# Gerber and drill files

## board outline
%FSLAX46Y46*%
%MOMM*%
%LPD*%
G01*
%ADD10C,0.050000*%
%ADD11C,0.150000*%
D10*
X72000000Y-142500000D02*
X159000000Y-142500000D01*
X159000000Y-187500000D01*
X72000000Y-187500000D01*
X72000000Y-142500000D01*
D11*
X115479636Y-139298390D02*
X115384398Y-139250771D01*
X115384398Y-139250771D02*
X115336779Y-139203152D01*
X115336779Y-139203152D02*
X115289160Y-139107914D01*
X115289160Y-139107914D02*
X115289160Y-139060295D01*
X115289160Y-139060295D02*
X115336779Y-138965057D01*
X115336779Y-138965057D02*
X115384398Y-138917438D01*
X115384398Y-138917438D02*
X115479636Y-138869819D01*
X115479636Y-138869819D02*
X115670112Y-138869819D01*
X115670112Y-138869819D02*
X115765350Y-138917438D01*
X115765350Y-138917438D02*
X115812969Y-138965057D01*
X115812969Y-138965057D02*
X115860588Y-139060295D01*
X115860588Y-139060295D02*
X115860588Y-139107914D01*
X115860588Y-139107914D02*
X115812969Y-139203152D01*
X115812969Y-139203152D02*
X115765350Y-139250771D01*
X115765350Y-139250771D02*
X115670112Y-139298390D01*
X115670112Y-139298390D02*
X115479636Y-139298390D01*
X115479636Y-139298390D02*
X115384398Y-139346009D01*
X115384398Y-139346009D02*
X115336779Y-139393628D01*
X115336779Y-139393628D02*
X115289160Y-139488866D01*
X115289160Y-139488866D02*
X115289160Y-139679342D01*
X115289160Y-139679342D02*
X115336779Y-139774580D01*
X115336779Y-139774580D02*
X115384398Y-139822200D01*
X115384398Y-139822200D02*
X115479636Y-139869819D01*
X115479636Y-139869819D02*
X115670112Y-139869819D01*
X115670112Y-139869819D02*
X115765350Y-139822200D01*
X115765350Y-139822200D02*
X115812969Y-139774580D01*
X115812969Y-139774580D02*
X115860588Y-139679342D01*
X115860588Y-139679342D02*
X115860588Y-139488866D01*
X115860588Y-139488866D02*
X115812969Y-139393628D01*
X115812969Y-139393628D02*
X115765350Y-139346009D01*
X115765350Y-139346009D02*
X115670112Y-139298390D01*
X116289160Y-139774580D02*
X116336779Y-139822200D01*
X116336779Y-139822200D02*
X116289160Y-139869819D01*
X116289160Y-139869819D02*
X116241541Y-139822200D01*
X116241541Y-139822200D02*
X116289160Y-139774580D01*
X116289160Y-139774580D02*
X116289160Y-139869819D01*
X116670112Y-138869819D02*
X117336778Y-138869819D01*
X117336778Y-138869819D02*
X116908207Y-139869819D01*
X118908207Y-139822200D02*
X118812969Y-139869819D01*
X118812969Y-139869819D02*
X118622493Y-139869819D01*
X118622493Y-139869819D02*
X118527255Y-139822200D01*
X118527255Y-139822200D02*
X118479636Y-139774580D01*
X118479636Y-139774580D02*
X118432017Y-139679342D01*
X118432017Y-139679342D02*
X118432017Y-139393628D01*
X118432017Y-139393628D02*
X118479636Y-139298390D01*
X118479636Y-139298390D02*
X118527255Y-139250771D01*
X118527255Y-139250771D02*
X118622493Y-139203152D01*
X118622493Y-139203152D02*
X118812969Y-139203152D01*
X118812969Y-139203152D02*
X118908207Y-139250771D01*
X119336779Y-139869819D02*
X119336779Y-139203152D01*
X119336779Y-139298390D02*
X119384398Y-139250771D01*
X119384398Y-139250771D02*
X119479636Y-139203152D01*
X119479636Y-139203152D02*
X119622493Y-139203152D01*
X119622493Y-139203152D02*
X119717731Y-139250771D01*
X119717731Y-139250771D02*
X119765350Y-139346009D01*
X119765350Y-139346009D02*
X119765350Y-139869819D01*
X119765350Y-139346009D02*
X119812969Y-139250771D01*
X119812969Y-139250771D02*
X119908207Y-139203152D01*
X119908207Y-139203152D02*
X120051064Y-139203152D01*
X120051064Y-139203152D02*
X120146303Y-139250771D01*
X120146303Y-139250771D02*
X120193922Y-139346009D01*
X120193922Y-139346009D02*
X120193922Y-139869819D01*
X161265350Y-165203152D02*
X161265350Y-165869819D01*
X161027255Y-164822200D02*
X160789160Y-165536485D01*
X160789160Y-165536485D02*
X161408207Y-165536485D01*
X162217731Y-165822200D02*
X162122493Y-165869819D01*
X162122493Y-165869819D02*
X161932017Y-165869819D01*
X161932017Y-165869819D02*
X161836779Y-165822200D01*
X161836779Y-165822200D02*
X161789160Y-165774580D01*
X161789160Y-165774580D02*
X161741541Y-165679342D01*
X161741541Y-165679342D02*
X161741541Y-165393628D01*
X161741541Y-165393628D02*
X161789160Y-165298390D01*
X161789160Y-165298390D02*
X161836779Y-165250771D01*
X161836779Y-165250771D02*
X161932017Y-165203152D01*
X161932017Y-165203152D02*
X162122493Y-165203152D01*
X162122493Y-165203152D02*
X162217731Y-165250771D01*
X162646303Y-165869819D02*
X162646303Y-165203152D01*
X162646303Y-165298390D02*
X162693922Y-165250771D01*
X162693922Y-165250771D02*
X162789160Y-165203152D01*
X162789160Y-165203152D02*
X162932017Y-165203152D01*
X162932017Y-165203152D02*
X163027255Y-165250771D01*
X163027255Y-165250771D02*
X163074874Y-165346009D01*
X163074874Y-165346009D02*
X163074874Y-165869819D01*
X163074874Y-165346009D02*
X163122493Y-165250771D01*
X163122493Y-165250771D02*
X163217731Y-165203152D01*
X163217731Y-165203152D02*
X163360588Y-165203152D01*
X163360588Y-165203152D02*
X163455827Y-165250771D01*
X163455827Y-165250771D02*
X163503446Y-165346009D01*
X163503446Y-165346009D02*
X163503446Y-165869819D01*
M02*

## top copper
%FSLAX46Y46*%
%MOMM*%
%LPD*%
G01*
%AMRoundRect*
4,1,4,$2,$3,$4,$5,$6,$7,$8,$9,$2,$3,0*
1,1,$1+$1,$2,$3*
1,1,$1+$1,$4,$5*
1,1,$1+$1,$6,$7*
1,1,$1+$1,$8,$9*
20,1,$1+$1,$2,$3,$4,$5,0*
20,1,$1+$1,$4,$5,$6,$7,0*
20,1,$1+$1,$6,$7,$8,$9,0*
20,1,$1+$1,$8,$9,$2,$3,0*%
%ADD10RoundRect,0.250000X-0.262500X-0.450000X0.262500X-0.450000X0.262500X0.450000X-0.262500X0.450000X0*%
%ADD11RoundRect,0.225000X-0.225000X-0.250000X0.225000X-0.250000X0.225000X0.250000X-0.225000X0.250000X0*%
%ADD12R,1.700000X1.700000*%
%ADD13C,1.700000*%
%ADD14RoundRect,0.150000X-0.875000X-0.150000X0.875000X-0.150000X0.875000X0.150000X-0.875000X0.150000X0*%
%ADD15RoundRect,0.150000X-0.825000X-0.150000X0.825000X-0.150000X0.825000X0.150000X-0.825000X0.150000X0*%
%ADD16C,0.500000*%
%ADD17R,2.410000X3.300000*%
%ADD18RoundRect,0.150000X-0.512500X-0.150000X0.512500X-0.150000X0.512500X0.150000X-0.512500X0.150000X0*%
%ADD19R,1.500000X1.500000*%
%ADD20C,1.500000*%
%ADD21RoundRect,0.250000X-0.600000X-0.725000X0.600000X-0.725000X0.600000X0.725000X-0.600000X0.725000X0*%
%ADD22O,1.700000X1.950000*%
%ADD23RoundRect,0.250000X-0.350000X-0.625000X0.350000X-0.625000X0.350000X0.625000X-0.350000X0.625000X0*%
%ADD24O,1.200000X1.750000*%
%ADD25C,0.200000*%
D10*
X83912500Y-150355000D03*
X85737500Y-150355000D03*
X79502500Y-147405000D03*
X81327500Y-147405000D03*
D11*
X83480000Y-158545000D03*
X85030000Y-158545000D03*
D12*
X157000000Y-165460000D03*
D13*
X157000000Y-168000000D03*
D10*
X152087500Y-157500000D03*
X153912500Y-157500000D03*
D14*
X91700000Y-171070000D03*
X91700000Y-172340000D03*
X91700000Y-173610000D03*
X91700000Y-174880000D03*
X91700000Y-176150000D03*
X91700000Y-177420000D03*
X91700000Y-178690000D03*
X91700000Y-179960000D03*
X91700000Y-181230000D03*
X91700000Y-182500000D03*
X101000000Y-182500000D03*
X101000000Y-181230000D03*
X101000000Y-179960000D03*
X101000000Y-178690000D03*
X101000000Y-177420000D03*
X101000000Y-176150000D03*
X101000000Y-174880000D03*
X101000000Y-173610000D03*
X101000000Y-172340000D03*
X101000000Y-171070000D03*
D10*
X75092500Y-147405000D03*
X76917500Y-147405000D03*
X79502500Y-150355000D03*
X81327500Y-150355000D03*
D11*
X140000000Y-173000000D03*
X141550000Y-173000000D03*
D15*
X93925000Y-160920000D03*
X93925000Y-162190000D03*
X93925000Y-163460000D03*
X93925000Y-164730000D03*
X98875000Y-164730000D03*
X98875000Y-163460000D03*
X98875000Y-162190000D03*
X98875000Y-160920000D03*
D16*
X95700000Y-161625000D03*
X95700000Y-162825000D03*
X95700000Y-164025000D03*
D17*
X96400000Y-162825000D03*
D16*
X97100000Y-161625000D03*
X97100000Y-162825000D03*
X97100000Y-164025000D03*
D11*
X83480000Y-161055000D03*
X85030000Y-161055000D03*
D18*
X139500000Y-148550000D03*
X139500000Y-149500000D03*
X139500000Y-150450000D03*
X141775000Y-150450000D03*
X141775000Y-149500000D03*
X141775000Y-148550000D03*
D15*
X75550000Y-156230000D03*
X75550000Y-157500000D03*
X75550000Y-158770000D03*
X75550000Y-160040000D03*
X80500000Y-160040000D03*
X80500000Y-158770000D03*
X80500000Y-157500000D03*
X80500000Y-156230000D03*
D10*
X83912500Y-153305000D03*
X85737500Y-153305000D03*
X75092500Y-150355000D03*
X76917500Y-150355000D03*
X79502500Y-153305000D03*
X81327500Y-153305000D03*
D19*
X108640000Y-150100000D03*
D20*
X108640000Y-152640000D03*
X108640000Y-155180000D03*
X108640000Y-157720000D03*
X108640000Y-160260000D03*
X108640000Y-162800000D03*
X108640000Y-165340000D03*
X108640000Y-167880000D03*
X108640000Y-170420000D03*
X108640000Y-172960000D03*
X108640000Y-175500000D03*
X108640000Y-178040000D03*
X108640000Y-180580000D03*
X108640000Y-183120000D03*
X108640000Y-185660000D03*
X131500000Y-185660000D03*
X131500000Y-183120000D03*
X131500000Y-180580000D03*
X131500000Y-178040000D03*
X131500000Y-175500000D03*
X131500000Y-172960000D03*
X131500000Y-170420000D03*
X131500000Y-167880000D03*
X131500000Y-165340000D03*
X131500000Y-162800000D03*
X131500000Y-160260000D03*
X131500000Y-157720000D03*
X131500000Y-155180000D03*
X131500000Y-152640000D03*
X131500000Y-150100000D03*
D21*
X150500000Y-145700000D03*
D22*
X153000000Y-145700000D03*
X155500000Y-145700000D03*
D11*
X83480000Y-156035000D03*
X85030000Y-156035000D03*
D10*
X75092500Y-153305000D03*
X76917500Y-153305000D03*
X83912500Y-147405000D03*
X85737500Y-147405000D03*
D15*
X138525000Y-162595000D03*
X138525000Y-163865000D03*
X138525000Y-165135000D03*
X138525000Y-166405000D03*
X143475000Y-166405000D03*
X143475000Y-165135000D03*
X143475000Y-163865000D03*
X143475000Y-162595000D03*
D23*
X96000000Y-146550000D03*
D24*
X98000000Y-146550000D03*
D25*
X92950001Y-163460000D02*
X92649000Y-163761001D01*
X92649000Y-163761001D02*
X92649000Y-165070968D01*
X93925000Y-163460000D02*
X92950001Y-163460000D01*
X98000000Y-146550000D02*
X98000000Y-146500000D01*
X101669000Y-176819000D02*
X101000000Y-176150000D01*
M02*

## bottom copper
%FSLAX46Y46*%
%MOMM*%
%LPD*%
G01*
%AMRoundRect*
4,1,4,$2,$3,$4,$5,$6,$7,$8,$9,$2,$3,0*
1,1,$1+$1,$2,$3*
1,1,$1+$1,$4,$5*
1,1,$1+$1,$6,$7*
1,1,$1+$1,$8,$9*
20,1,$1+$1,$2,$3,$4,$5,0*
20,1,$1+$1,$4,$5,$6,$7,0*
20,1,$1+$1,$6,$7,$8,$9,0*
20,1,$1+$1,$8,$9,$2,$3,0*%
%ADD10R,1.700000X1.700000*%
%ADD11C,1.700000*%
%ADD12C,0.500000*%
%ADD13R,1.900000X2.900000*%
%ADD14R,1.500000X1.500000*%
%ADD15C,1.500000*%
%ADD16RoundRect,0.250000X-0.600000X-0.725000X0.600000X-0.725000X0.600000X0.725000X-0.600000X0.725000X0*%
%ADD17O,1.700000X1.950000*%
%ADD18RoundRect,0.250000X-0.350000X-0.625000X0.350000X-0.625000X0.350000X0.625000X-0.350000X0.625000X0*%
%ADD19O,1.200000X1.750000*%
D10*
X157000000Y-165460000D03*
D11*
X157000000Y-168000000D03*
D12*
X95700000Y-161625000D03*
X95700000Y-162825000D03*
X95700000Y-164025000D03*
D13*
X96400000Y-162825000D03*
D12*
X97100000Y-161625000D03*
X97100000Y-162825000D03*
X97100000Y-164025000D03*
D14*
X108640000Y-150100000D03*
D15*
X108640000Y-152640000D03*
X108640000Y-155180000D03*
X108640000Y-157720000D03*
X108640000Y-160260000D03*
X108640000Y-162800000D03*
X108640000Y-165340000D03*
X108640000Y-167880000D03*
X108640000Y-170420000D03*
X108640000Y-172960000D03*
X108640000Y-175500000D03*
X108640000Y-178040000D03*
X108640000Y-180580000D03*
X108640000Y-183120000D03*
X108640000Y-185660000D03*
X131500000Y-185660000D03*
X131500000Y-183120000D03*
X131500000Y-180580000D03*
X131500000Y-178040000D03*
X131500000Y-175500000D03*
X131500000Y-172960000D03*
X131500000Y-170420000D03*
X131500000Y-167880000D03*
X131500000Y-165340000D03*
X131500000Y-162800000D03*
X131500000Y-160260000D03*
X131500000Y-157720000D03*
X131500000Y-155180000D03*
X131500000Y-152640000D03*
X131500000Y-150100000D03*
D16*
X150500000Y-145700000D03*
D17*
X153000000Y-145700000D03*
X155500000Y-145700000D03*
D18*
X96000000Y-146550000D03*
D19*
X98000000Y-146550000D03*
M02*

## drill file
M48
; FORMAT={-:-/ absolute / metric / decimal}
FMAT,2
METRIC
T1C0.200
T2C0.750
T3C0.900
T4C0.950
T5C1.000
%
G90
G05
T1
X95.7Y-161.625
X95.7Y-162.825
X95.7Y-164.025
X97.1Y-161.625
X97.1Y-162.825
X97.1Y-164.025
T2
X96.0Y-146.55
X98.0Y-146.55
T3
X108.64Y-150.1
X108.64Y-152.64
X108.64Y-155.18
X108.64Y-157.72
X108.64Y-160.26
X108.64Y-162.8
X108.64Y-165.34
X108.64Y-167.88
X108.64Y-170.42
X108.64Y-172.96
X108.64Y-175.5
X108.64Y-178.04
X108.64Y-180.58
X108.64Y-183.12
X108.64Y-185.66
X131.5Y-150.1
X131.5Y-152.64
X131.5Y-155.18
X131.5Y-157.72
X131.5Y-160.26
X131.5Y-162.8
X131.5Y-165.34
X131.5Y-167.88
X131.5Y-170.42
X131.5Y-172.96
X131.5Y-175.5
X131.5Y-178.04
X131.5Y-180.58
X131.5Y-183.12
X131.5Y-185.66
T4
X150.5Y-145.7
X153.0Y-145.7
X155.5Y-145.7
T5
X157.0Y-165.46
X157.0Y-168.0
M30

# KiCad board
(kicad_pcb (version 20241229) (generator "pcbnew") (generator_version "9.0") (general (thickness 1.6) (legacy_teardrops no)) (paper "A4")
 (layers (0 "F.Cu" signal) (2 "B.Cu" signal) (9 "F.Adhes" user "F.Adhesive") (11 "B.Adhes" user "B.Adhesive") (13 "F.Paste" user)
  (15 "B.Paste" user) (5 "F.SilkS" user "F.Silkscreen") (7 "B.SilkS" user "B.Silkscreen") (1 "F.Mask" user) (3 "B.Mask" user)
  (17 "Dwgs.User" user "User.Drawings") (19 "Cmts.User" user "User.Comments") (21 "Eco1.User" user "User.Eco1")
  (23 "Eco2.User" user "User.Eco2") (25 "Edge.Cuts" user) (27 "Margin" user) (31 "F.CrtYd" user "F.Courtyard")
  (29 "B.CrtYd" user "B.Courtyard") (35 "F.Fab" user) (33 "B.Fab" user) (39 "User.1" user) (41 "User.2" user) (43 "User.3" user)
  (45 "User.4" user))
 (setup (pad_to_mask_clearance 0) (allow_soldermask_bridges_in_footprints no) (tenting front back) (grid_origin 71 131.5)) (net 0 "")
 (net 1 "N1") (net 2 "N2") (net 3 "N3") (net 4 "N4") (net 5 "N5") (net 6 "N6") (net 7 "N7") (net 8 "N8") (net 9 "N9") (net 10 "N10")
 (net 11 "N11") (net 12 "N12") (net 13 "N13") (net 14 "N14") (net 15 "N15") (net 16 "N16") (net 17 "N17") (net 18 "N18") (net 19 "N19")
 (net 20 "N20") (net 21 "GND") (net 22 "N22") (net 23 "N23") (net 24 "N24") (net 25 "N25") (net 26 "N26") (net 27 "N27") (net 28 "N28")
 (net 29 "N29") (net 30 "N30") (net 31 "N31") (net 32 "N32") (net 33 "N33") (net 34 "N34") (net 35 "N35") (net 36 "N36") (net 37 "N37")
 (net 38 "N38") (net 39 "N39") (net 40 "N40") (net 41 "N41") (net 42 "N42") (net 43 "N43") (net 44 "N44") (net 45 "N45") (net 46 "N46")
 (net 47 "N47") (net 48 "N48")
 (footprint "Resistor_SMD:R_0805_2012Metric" (layer "F.Cu") (at 84.825 150.355)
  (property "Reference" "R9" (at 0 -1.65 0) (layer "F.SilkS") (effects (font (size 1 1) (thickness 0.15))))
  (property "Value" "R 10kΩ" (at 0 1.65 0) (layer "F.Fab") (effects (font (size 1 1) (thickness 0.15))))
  (pad "1" smd roundrect (at -0.9125 0) (size 1.025 1.4) (layers "F.Cu" "F.Mask" "F.Paste") (roundrect_rratio 0.243902) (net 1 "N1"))
  (pad "2" smd roundrect (at 0.9125 0) (size 1.025 1.4) (layers "F.Cu" "F.Mask" "F.Paste") (roundrect_rratio 0.243902) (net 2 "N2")))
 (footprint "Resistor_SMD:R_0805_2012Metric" (layer "F.Cu") (at 80.415 147.405)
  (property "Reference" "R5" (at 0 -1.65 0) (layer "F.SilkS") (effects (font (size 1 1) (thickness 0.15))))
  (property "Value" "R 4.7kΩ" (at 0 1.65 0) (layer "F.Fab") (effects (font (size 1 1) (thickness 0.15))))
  (pad "1" smd roundrect (at -0.9125 0) (size 1.025 1.4) (layers "F.Cu" "F.Mask" "F.Paste") (roundrect_rratio 0.243902) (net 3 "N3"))
  (pad "2" smd roundrect (at 0.9125 0) (size 1.025 1.4) (layers "F.Cu" "F.Mask" "F.Paste") (roundrect_rratio 0.243902) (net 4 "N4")))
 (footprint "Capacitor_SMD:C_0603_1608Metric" (layer "F.Cu") (at 84.255 158.545)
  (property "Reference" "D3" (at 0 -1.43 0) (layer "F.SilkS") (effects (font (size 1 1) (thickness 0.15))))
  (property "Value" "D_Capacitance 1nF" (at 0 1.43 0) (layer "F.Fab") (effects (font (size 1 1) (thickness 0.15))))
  (pad "1" smd roundrect (at -0.775 0) (size 0.9 0.95) (layers "F.Cu" "F.Mask" "F.Paste") (roundrect_rratio 0.25) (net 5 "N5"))
  (pad "2" smd roundrect (at 0.775 0) (size 0.9 0.95) (layers "F.Cu" "F.Mask" "F.Paste") (roundrect_rratio 0.25) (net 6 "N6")))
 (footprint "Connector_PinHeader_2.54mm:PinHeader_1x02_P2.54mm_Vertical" (layer "F.Cu") (at 157 165.46)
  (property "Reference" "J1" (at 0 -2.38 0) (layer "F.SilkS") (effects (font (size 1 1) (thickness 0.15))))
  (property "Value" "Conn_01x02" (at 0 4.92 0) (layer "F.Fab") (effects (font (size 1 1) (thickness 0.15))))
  (pad "1" thru_hole rect (at 0 0) (size 1.7 1.7) (drill 1) (layers "*.Cu" "*.Mask") (remove_unused_layers no) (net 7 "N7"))
  (pad "2" thru_hole circle (at 0 2.54) (size 1.7 1.7) (drill 1) (layers "*.Cu" "*.Mask") (remove_unused_layers no) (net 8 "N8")))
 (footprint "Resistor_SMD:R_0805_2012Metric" (layer "F.Cu") (at 153 157.5)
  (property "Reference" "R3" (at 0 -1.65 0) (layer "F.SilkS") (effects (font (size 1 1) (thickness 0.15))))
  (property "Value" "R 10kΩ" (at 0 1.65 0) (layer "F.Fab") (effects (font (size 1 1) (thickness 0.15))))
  (pad "1" smd roundrect (at -0.9125 0) (size 1.025 1.4) (layers "F.Cu" "F.Mask" "F.Paste") (roundrect_rratio 0.243902) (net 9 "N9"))
  (pad "2" smd roundrect (at 0.9125 0) (size 1.025 1.4) (layers "F.Cu" "F.Mask" "F.Paste") (roundrect_rratio 0.243902) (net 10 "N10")))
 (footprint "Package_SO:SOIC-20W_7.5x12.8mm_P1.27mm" (layer "F.Cu") (at 96.35 176.785)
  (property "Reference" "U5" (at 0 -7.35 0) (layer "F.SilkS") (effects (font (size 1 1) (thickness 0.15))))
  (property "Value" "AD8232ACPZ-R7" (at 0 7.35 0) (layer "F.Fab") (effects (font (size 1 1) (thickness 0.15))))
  (pad "1" smd roundrect (at -4.65 -5.715) (size 2.05 0.6) (layers "F.Cu" "F.Mask" "F.Paste") (roundrect_rratio 0.25) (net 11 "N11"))
  (pad "2" smd roundrect (at -4.65 -4.445) (size 2.05 0.6) (layers "F.Cu" "F.Mask" "F.Paste") (roundrect_rratio 0.25) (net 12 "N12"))
  (pad "3" smd roundrect (at -4.65 -3.175) (size 2.05 0.6) (layers "F.Cu" "F.Mask" "F.Paste") (roundrect_rratio 0.25) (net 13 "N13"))
  (pad "4" smd roundrect (at -4.65 -1.905) (size 2.05 0.6) (layers "F.Cu" "F.Mask" "F.Paste") (roundrect_rratio 0.25) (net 5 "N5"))
  (pad "5" smd roundrect (at -4.65 -0.635) (size 2.05 0.6) (layers "F.Cu" "F.Mask" "F.Paste") (roundrect_rratio 0.25) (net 6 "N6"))
  (pad "6" smd roundrect (at -4.65 0.635) (size 2.05 0.6) (layers "F.Cu" "F.Mask" "F.Paste") (roundrect_rratio 0.25) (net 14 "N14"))
  (pad "7" smd roundrect (at -4.65 1.905) (size 2.05 0.6) (layers "F.Cu" "F.Mask" "F.Paste") (roundrect_rratio 0.25) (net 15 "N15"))
  (pad "8" smd roundrect (at -4.65 3.175) (size 2.05 0.6) (layers "F.Cu" "F.Mask" "F.Paste") (roundrect_rratio 0.25) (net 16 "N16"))
  (pad "9" smd roundrect (at -4.65 4.445) (size 2.05 0.6) (layers "F.Cu" "F.Mask" "F.Paste") (roundrect_rratio 0.25) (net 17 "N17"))
  (pad "10" smd roundrect (at -4.65 5.715) (size 2.05 0.6) (layers "F.Cu" "F.Mask" "F.Paste") (roundrect_rratio 0.25) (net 9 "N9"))
  (pad "11" smd roundrect (at 4.65 5.715) (size 2.05 0.6) (layers "F.Cu" "F.Mask" "F.Paste") (roundrect_rratio 0.25) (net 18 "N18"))
  (pad "12" smd roundrect (at 4.65 4.445) (size 2.05 0.6) (layers "F.Cu" "F.Mask" "F.Paste") (roundrect_rratio 0.25) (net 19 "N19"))
  (pad "13" smd roundrect (at 4.65 3.175) (size 2.05 0.6) (layers "F.Cu" "F.Mask" "F.Paste") (roundrect_rratio 0.25) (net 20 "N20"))
  (pad "14" smd roundrect (at 4.65 1.905) (size 2.05 0.6) (layers "F.Cu" "F.Mask" "F.Paste") (roundrect_rratio 0.25) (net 16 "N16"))
  (pad "15" smd roundrect (at 4.65 0.635) (size 2.05 0.6) (layers "F.Cu" "F.Mask" "F.Paste") (roundrect_rratio 0.25) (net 16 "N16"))
  (pad "16" smd roundrect (at 4.65 -0.635) (size 2.05 0.6) (layers "F.Cu" "F.Mask" "F.Paste") (roundrect_rratio 0.25) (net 10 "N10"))
  (pad "17" smd roundrect (at 4.65 -1.905) (size 2.05 0.6) (layers "F.Cu" "F.Mask" "F.Paste") (roundrect_rratio 0.25) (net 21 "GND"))
  (pad "18" smd roundrect (at 4.65 -3.175) (size 2.05 0.6) (layers "F.Cu" "F.Mask" "F.Paste") (roundrect_rratio 0.25) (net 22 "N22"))
  (pad "19" smd roundrect (at 4.65 -4.445) (size 2.05 0.6) (layers "F.Cu" "F.Mask" "F.Paste") (roundrect_rratio 0.25) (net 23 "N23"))
  (pad "20" smd roundrect (at 4.65 -5.715) (size 2.05 0.6) (layers "F.Cu" "F.Mask" "F.Paste") (roundrect_rratio 0.25) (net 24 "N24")))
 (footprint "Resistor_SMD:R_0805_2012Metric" (layer "F.Cu") (at 76.005 147.405)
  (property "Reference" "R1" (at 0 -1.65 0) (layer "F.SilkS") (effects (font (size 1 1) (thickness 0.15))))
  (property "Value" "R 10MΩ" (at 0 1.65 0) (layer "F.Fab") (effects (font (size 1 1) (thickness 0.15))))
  (pad "1" smd roundrect (at -0.9125 0) (size 1.025 1.4) (layers "F.Cu" "F.Mask" "F.Paste") (roundrect_rratio 0.243902) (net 13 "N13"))
  (pad "2" smd roundrect (at 0.9125 0) (size 1.025 1.4) (layers "F.Cu" "F.Mask" "F.Paste") (roundrect_rratio 0.243902) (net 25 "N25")))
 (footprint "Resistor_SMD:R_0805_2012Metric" (layer "F.Cu") (at 80.415 150.355)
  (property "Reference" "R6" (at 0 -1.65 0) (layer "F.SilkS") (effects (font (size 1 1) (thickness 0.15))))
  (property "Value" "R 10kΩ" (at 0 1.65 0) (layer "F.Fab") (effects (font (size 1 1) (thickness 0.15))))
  (pad "1" smd roundrect (at -0.9125 0) (size 1.025 1.4) (layers "F.Cu" "F.Mask" "F.Paste") (roundrect_rratio 0.243902) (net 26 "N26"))
  (pad "2" smd roundrect (at 0.9125 0) (size 1.025 1.4) (layers "F.Cu" "F.Mask" "F.Paste") (roundrect_rratio 0.243902) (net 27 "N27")))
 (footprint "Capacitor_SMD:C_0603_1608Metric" (layer "F.Cu") (at 140.775 173)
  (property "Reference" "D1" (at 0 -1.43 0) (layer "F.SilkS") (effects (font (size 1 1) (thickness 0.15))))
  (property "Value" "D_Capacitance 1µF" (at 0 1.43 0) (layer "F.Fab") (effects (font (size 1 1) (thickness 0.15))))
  (pad "1" smd roundrect (at -0.775 0) (size 0.9 0.95) (layers "F.Cu" "F.Mask" "F.Paste") (roundrect_rratio 0.25) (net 21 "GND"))
  (pad "2" smd roundrect (at 0.775 0) (size 0.9 0.95) (layers "F.Cu" "F.Mask" "F.Paste") (roundrect_rratio 0.25) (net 10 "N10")))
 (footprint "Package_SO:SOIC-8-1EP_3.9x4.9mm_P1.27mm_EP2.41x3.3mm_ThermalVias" (layer "F.Cu") (at 96.4 162.825)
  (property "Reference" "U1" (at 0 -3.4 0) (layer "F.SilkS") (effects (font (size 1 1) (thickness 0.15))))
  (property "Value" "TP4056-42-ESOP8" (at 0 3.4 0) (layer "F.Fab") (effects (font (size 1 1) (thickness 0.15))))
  (pad "" smd roundrect (at -0.6 -0.825) (size 1.01 1.38) (layers "F.Paste") (roundrect_rratio 0.247525))
  (pad "" smd roundrect (at -0.6 0.825) (size 1.01 1.38) (layers "F.Paste") (roundrect_rratio 0.247525))
  (pad "" smd roundrect (at 0.6 -0.825) (size 1.01 1.38) (layers "F.Paste") (roundrect_rratio 0.247525))
  (pad "" smd roundrect (at 0.6 0.825) (size 1.01 1.38) (layers "F.Paste") (roundrect_rratio 0.247525))
  (pad "1" smd roundrect (at -2.475 -1.905) (size 1.95 0.6) (layers "F.Cu" "F.Mask" "F.Paste") (roundrect_rratio 0.25) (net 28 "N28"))
  (pad "2" smd roundrect (at -2.475 -0.635) (size 1.95 0.6) (layers "F.Cu" "F.Mask" "F.Paste") (roundrect_rratio 0.25) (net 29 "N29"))
  (pad "3" smd roundrect (at -2.475 0.635) (size 1.95 0.6) (layers "F.Cu" "F.Mask" "F.Paste") (roundrect_rratio 0.25) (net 21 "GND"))
  (pad "4" smd roundrect (at -2.475 1.905) (size 1.95 0.6) (layers "F.Cu" "F.Mask" "F.Paste") (roundrect_rratio 0.25) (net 21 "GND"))
  (pad "5" smd roundrect (at 2.475 1.905) (size 1.95 0.6) (layers "F.Cu" "F.Mask" "F.Paste") (roundrect_rratio 0.25) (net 21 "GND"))
  (pad "6" smd roundrect (at 2.475 0.635) (size 1.95 0.6) (layers "F.Cu" "F.Mask" "F.Paste") (roundrect_rratio 0.25) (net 27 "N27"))
  (pad "7" smd roundrect (at 2.475 -0.635) (size 1.95 0.6) (layers "F.Cu" "F.Mask" "F.Paste") (roundrect_rratio 0.25) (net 4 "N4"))
  (pad "8" smd roundrect (at 2.475 -1.905) (size 1.95 0.6) (layers "F.Cu" "F.Mask" "F.Paste") (roundrect_rratio 0.25) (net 21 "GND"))
  (pad "9" thru_hole circle (at -0.7 -1.2) (size 0.5 0.5) (drill 0.2) (layers "*.Cu") (remove_unused_layers no) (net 21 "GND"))
  (pad "9" thru_hole circle (at -0.7 0) (size 0.5 0.5) (drill 0.2) (layers "*.Cu") (remove_unused_layers no) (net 21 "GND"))
  (pad "9" thru_hole circle (at -0.7 1.2) (size 0.5 0.5) (drill 0.2) (layers "*.Cu") (remove_unused_layers no) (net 21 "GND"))
  (pad "9" smd rect (at 0 0) (size 1.9 2.9) (layers "B.Cu") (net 21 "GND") (zone_connect 2))
  (pad "9" smd rect (at 0 0) (size 2.41 3.3) (layers "F.Cu" "F.Mask") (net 21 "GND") (zone_connect 2))
  (pad "9" thru_hole circle (at 0.7 -1.2) (size 0.5 0.5) (drill 0.2) (layers "*.Cu") (remove_unused_layers no) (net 21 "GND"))
  (pad "9" thru_hole circle (at 0.7 0) (size 0.5 0.5) (drill 0.2) (layers "*.Cu") (remove_unused_layers no) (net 21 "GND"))
  (pad "9" thru_hole circle (at 0.7 1.2) (size 0.5 0.5) (drill 0.2) (layers "*.Cu") (remove_unused_layers no) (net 21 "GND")))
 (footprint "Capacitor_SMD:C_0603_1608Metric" (layer "F.Cu") (at 84.255 161.055)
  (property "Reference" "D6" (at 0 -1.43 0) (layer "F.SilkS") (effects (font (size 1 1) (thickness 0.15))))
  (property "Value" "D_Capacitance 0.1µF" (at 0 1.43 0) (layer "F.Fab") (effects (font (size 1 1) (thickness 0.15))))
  (pad "1" smd roundrect (at -0.775 0) (size 0.9 0.95) (layers "F.Cu" "F.Mask" "F.Paste") (roundrect_rratio 0.25) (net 25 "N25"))
  (pad "2" smd roundrect (at 0.775 0) (size 0.9 0.95) (layers "F.Cu" "F.Mask" "F.Paste") (roundrect_rratio 0.25) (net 22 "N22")))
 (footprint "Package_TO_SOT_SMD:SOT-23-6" (layer "F.Cu") (at 140.6375 149.5)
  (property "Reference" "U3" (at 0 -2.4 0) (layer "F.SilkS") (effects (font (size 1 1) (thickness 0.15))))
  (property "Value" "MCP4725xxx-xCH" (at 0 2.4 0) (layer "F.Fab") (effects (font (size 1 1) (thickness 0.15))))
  (pad "1" smd roundrect (at -1.1375 -0.95) (size 1.325 0.6) (layers "F.Cu" "F.Mask" "F.Paste") (roundrect_rratio 0.25) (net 1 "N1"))
  (pad "2" smd roundrect (at -1.1375 0) (size 1.325 0.6) (layers "F.Cu" "F.Mask" "F.Paste") (roundrect_rratio 0.25) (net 21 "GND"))
  (pad "3" smd roundrect (at -1.1375 0.95) (size 1.325 0.6) (layers "F.Cu" "F.Mask" "F.Paste") (roundrect_rratio 0.25) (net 21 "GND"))
  (pad "4" smd roundrect (at 1.1375 0.95) (size 1.325 0.6) (layers "F.Cu" "F.Mask" "F.Paste") (roundrect_rratio 0.25) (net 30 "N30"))
  (pad "5" smd roundrect (at 1.1375 0) (size 1.325 0.6) (layers "F.Cu" "F.Mask" "F.Paste") (roundrect_rratio 0.25) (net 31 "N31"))
  (pad "6" smd roundrect (at 1.1375 -0.95) (size 1.325 0.6) (layers "F.Cu" "F.Mask" "F.Paste") (roundrect_rratio 0.25) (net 21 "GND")))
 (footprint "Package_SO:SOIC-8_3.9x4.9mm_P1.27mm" (layer "F.Cu") (at 78.025 158.135)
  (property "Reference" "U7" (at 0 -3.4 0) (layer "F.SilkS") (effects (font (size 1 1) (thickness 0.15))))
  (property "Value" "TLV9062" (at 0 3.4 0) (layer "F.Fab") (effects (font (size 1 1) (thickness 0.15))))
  (pad "1" smd roundrect (at -2.475 -1.905) (size 1.95 0.6) (layers "F.Cu" "F.Mask" "F.Paste") (roundrect_rratio 0.25) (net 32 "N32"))
  (pad "2" smd roundrect (at -2.475 -0.635) (size 1.95 0.6) (layers "F.Cu" "F.Mask" "F.Paste") (roundrect_rratio 0.25) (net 2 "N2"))
  (pad "3" smd roundrect (at -2.475 0.635) (size 1.95 0.6) (layers "F.Cu" "F.Mask" "F.Paste") (roundrect_rratio 0.25) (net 21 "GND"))
  (pad "4" smd roundrect (at -2.475 1.905) (size 1.95 0.6) (layers "F.Cu" "F.Mask" "F.Paste") (roundrect_rratio 0.25))
  (pad "5" smd roundrect (at 2.475 1.905) (size 1.95 0.6) (layers "F.Cu" "F.Mask" "F.Paste") (roundrect_rratio 0.25))
  (pad "6" smd roundrect (at 2.475 0.635) (size 1.95 0.6) (layers "F.Cu" "F.Mask" "F.Paste") (roundrect_rratio 0.25))
  (pad "7" smd roundrect (at 2.475 -0.635) (size 1.95 0.6) (layers "F.Cu" "F.Mask" "F.Paste") (roundrect_rratio 0.25))
  (pad "8" smd roundrect (at 2.475 -1.905) (size 1.95 0.6) (layers "F.Cu" "F.Mask" "F.Paste") (roundrect_rratio 0.25)))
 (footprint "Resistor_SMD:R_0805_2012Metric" (layer "F.Cu") (at 84.825 153.305)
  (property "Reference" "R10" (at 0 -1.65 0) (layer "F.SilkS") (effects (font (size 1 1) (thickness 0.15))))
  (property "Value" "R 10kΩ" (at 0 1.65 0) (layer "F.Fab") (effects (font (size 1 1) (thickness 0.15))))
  (pad "1" smd roundrect (at -0.9125 0) (size 1.025 1.4) (layers "F.Cu" "F.Mask" "F.Paste") (roundrect_rratio 0.243902) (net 1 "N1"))
  (pad "2" smd roundrect (at 0.9125 0) (size 1.025 1.4) (layers "F.Cu" "F.Mask" "F.Paste") (roundrect_rratio 0.243902) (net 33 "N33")))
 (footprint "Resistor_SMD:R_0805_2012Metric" (layer "F.Cu") (at 76.005 150.355)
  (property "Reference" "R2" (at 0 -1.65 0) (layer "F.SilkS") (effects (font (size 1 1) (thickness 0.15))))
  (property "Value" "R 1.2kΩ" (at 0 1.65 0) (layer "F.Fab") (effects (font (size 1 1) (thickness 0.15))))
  (pad "1" smd roundrect (at -0.9125 0) (size 1.025 1.4) (layers "F.Cu" "F.Mask" "F.Paste") (roundrect_rratio 0.243902) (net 29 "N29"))
  (pad "2" smd roundrect (at 0.9125 0) (size 1.025 1.4) (layers "F.Cu" "F.Mask" "F.Paste") (roundrect_rratio 0.243902) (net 21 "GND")))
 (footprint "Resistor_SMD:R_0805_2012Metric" (layer "F.Cu") (at 80.415 153.305)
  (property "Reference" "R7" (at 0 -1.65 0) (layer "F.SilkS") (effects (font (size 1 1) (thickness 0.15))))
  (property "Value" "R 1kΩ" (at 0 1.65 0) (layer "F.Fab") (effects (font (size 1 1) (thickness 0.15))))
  (pad "1" smd roundrect (at -0.9125 0) (size 1.025 1.4) (layers "F.Cu" "F.Mask" "F.Paste") (roundrect_rratio 0.243902) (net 8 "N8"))
  (pad "2" smd roundrect (at 0.9125 0) (size 1.025 1.4) (layers "F.Cu" "F.Mask" "F.Paste") (roundrect_rratio 0.243902) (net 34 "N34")))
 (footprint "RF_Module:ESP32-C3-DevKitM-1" (layer "F.Cu") (at 108.64 150.1)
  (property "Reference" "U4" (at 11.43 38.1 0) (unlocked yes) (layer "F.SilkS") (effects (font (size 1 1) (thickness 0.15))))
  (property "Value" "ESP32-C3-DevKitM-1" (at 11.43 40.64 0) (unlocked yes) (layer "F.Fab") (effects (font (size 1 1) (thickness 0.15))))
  (pad "1" thru_hole rect (at 0 0) (size 1.5 1.5) (drill 0.9) (layers "*.Cu" "*.Mask") (remove_unused_layers yes) (keep_end_layers yes)
   (zone_layer_connections) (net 21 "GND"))
  (pad "2" thru_hole circle (at 0 2.54) (size 1.5 1.5) (drill 0.9) (layers "*.Cu" "*.Mask") (remove_unused_layers yes) (keep_end_layers yes)
   (zone_layer_connections) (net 21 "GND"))
  (pad "3" thru_hole circle (at 0 5.08) (size 1.5 1.5) (drill 0.9) (layers "*.Cu" "*.Mask") (remove_unused_layers yes) (keep_end_layers yes)
   (zone_layer_connections) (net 21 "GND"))
  (pad "4" thru_hole circle (at 0 7.62) (size 1.5 1.5) (drill 0.9) (layers "*.Cu" "*.Mask") (remove_unused_layers yes) (keep_end_layers yes)
   (zone_layer_connections) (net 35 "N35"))
  (pad "5" thru_hole circle (at 0 10.16) (size 1.5 1.5) (drill 0.9) (layers "*.Cu" "*.Mask") (remove_unused_layers yes)
   (keep_end_layers yes) (zone_layer_connections) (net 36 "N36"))
  (pad "6" thru_hole circle (at 0 12.7) (size 1.5 1.5) (drill 0.9) (layers "*.Cu" "*.Mask") (remove_unused_layers yes) (keep_end_layers yes)
   (zone_layer_connections) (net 21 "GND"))
  (pad "7" thru_hole circle (at 0 15.24) (size 1.5 1.5) (drill 0.9) (layers "*.Cu" "*.Mask") (remove_unused_layers yes)
   (keep_end_layers yes) (zone_layer_connections) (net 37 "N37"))
  (pad "8" thru_hole circle (at 0 17.78) (size 1.5 1.5) (drill 0.9) (layers "*.Cu" "*.Mask") (remove_unused_layers yes)
   (keep_end_layers yes) (zone_layer_connections) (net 21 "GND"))
  (pad "9" thru_hole circle (at 0 20.32) (size 1.5 1.5) (drill 0.9) (layers "*.Cu" "*.Mask") (remove_unused_layers yes)
   (keep_end_layers yes) (zone_layer_connections) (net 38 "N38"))
  (pad "10" thru_hole circle (at 0 22.86) (size 1.5 1.5) (drill 0.9) (layers "*.Cu" "*.Mask") (remove_unused_layers yes)
   (keep_end_layers yes) (zone_layer_connections) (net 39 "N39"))
  (pad "11" thru_hole circle (at 0 25.4) (size 1.5 1.5) (drill 0.9) (layers "*.Cu" "*.Mask") (remove_unused_layers yes)
   (keep_end_layers yes) (zone_layer_connections) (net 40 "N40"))
  (pad "12" thru_hole circle (at 0 27.94) (size 1.5 1.5) (drill 0.9) (layers "*.Cu" "*.Mask") (remove_unused_layers yes)
   (keep_end_layers yes) (zone_layer_connections) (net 21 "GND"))
  (pad "13" thru_hole circle (at 0 30.48) (size 1.5 1.5) (drill 0.9) (layers "*.Cu" "*.Mask") (remove_unused_layers yes)
   (keep_end_layers yes) (zone_layer_connections) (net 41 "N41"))
  (pad "14" thru_hole circle (at 0 33.02) (size 1.5 1.5) (drill 0.9) (layers "*.Cu" "*.Mask") (remove_unused_layers yes)
   (keep_end_layers yes) (zone_layer_connections) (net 41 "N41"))
  (pad "15" thru_hole circle (at 0 35.56) (size 1.5 1.5) (drill 0.9) (layers "*.Cu" "*.Mask") (remove_unused_layers yes)
   (keep_end_layers yes) (zone_layer_connections) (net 21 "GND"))
  (pad "16" thru_hole circle (at 22.86 35.56) (size 1.5 1.5) (drill 0.9) (layers "*.Cu" "*.Mask") (remove_unused_layers yes)
   (keep_end_layers yes) (zone_layer_connections) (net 21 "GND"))
  (pad "17" thru_hole circle (at 22.86 33.02) (size 1.5 1.5) (drill 0.9) (layers "*.Cu" "*.Mask") (remove_unused_layers yes)
   (keep_end_layers yes) (zone_layer_connections) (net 9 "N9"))
  (pad "18" thru_hole circle (at 22.86 30.48) (size 1.5 1.5) (drill 0.9) (layers "*.Cu" "*.Mask") (remove_unused_layers yes)
   (keep_end_layers yes) (zone_layer_connections) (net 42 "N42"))
  (pad "19" thru_hole circle (at 22.86 27.94) (size 1.5 1.5) (drill 0.9) (layers "*.Cu" "*.Mask") (remove_unused_layers yes)
   (keep_end_layers yes) (zone_layer_connections) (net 21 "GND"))
  (pad "20" thru_hole circle (at 22.86 25.4) (size 1.5 1.5) (drill 0.9) (layers "*.Cu" "*.Mask") (remove_unused_layers yes)
   (keep_end_layers yes) (zone_layer_connections) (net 31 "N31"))
  (pad "21" thru_hole circle (at 22.86 22.86) (size 1.5 1.5) (drill 0.9) (layers "*.Cu" "*.Mask") (remove_unused_layers yes)
   (keep_end_layers yes) (zone_layer_connections) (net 30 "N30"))
  (pad "22" thru_hole circle (at 22.86 20.32) (size 1.5 1.5) (drill 0.9) (layers "*.Cu" "*.Mask") (remove_unused_layers yes)
   (keep_end_layers yes) (zone_layer_connections) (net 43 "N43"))
  (pad "23" thru_hole circle (at 22.86 17.78) (size 1.5 1.5) (drill 0.9) (layers "*.Cu" "*.Mask") (remove_unused_layers yes)
   (keep_end_layers yes) (zone_layer_connections) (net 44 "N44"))
  (pad "24" thru_hole circle (at 22.86 15.24) (size 1.5 1.5) (drill 0.9) (layers "*.Cu" "*.Mask") (remove_unused_layers yes)
   (keep_end_layers yes) (zone_layer_connections) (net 21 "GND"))
  (pad "25" thru_hole circle (at 22.86 12.7) (size 1.5 1.5) (drill 0.9) (layers "*.Cu" "*.Mask") (remove_unused_layers yes)
   (keep_end_layers yes) (zone_layer_connections) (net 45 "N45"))
  (pad "26" thru_hole circle (at 22.86 10.16) (size 1.5 1.5) (drill 0.9) (layers "*.Cu" "*.Mask") (remove_unused_layers yes)
   (keep_end_layers yes) (zone_layer_connections) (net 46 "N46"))
  (pad "27" thru_hole circle (at 22.86 7.62) (size 1.5 1.5) (drill 0.9) (layers "*.Cu" "*.Mask") (remove_unused_layers yes)
   (keep_end_layers yes) (zone_layer_connections) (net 21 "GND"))
  (pad "28" thru_hole circle (at 22.86 5.08) (size 1.5 1.5) (drill 0.9) (layers "*.Cu" "*.Mask") (remove_unused_layers yes)
   (keep_end_layers yes) (zone_layer_connections) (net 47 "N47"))
  (pad "29" thru_hole circle (at 22.86 2.54) (size 1.5 1.5) (drill 0.9) (layers "*.Cu" "*.Mask") (remove_unused_layers yes)
   (keep_end_layers yes) (zone_layer_connections) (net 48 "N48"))
  (pad "30" thru_hole circle (at 22.86 0) (size 1.5 1.5) (drill 0.9) (layers "*.Cu" "*.Mask") (remove_unused_layers yes)
   (keep_end_layers yes) (zone_layer_connections) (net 21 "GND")))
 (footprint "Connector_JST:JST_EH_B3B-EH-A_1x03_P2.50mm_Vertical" (layer "F.Cu") (at 150.5 145.7)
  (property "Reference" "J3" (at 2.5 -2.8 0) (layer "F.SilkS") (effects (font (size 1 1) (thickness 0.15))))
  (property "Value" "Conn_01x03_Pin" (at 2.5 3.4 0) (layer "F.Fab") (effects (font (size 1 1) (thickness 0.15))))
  (pad "1" thru_hole roundrect (at 0 0) (size 1.7 1.95) (drill 0.95) (layers "*.Cu" "*.Mask") (remove_unused_layers no)
   (roundrect_rratio 0.147059) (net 12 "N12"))
  (pad "2" thru_hole oval (at 2.5 0) (size 1.7 1.95) (drill 0.95) (layers "*.Cu" "*.Mask") (remove_unused_layers no) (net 13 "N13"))
  (pad "3" thru_hole oval (at 5 0) (size 1.7 1.95) (drill 0.95) (layers "*.Cu" "*.Mask") (remove_unused_layers no) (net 25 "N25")))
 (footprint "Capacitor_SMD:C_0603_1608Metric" (layer "F.Cu") (at 84.255 156.035)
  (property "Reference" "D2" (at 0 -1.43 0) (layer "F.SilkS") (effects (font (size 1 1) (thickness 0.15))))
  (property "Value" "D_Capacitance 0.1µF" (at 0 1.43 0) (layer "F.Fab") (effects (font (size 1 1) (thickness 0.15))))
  (pad "1" smd roundrect (at -0.775 0) (size 0.9 0.95) (layers "F.Cu" "F.Mask" "F.Paste") (roundrect_rratio 0.25) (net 25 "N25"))
  (pad "2" smd roundrect (at 0.775 0) (size 0.9 0.95) (layers "F.Cu" "F.Mask" "F.Paste") (roundrect_rratio 0.25) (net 16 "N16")))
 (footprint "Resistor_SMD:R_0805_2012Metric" (layer "F.Cu") (at 76.005 153.305)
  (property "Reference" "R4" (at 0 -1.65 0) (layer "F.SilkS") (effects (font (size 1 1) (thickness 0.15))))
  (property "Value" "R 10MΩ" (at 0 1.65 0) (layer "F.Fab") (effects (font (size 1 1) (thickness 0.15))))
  (pad "1" smd roundrect (at -0.9125 0) (size 1.025 1.4) (layers "F.Cu" "F.Mask" "F.Paste") (roundrect_rratio 0.243902) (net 12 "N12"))
  (pad "2" smd roundrect (at 0.9125 0) (size 1.025 1.4) (layers "F.Cu" "F.Mask" "F.Paste") (roundrect_rratio 0.243902) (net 25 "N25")))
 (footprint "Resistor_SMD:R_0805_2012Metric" (layer "F.Cu") (at 84.825 147.405)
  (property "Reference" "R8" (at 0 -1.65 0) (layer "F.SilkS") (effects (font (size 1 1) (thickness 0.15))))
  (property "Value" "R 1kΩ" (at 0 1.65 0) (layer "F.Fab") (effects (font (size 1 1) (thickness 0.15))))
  (pad "1" smd roundrect (at -0.9125 0) (size 1.025 1.4) (layers "F.Cu" "F.Mask" "F.Paste") (roundrect_rratio 0.243902) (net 7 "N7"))
  (pad "2" smd roundrect (at 0.9125 0) (size 1.025 1.4) (layers "F.Cu" "F.Mask" "F.Paste") (roundrect_rratio 0.243902) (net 32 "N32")))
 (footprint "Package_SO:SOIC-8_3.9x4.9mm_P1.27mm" (layer "F.Cu") (at 141 164.5)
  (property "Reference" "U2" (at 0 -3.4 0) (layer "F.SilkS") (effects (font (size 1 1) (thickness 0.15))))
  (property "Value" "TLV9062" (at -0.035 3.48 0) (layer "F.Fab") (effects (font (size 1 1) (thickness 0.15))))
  (pad "1" smd roundrect (at -2.475 -1.905) (size 1.95 0.6) (layers "F.Cu" "F.Mask" "F.Paste") (roundrect_rratio 0.25) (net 34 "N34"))
  (pad "2" smd roundrect (at -2.475 -0.635) (size 1.95 0.6) (layers "F.Cu" "F.Mask" "F.Paste") (roundrect_rratio 0.25) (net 34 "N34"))
  (pad "3" smd roundrect (at -2.475 0.635) (size 1.95 0.6) (layers "F.Cu" "F.Mask" "F.Paste") (roundrect_rratio 0.25) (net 33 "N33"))
  (pad "4" smd roundrect (at -2.475 1.905) (size 1.95 0.6) (layers "F.Cu" "F.Mask" "F.Paste") (roundrect_rratio 0.25))
  (pad "5" smd roundrect (at 2.475 1.905) (size 1.95 0.6) (layers "F.Cu" "F.Mask" "F.Paste") (roundrect_rratio 0.25))
  (pad "6" smd roundrect (at 2.475 0.635) (size 1.95 0.6) (layers "F.Cu" "F.Mask" "F.Paste") (roundrect_rratio 0.25))
  (pad "7" smd roundrect (at 2.475 -0.635) (size 1.95 0.6) (layers "F.Cu" "F.Mask" "F.Paste") (roundrect_rratio 0.25))
  (pad "8" smd roundrect (at 2.475 -1.905) (size 1.95 0.6) (layers "F.Cu" "F.Mask" "F.Paste") (roundrect_rratio 0.25)))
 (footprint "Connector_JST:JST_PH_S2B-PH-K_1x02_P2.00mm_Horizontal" (layer "F.Cu") (at 96 146.55)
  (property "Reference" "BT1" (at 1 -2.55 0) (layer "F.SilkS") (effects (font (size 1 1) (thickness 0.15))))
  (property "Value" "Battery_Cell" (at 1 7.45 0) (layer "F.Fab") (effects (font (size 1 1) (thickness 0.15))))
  (pad "1" thru_hole roundrect (at 0 0) (size 1.2 1.75) (drill 0.75) (layers "*.Cu" "*.Mask") (remove_unused_layers no)
   (roundrect_rratio 0.208333) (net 21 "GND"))
  (pad "2" thru_hole oval (at 2 0) (size 1.2 1.75) (drill 0.75) (layers "*.Cu" "*.Mask") (remove_unused_layers no) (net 28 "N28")))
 (gr_rect (start 72 142.5) (end 159 187.5) (stroke (width 0.05) (type solid)) (fill no) (layer "Edge.Cuts"))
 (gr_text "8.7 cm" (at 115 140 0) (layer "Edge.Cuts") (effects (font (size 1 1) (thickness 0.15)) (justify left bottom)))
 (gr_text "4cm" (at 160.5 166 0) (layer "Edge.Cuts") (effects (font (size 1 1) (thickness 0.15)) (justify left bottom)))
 (segment (start 92.950001 163.46) (end 92.649 163.761001) (width 0.2) (layer "F.Cu") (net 21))
 (segment (start 92.649 163.761001) (end 92.649 165.070968) (width 0.2) (layer "F.Cu") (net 21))
 (segment (start 93.925 163.46) (end 92.950001 163.46) (width 0.2) (layer "F.Cu") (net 21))
 (segment (start 98 146.55) (end 98 146.5) (width 0.2) (layer "F.Cu") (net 28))
 (segment (start 101.669 176.819) (end 101 176.15) (width 0.2) (layer "F.Cu") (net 10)))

